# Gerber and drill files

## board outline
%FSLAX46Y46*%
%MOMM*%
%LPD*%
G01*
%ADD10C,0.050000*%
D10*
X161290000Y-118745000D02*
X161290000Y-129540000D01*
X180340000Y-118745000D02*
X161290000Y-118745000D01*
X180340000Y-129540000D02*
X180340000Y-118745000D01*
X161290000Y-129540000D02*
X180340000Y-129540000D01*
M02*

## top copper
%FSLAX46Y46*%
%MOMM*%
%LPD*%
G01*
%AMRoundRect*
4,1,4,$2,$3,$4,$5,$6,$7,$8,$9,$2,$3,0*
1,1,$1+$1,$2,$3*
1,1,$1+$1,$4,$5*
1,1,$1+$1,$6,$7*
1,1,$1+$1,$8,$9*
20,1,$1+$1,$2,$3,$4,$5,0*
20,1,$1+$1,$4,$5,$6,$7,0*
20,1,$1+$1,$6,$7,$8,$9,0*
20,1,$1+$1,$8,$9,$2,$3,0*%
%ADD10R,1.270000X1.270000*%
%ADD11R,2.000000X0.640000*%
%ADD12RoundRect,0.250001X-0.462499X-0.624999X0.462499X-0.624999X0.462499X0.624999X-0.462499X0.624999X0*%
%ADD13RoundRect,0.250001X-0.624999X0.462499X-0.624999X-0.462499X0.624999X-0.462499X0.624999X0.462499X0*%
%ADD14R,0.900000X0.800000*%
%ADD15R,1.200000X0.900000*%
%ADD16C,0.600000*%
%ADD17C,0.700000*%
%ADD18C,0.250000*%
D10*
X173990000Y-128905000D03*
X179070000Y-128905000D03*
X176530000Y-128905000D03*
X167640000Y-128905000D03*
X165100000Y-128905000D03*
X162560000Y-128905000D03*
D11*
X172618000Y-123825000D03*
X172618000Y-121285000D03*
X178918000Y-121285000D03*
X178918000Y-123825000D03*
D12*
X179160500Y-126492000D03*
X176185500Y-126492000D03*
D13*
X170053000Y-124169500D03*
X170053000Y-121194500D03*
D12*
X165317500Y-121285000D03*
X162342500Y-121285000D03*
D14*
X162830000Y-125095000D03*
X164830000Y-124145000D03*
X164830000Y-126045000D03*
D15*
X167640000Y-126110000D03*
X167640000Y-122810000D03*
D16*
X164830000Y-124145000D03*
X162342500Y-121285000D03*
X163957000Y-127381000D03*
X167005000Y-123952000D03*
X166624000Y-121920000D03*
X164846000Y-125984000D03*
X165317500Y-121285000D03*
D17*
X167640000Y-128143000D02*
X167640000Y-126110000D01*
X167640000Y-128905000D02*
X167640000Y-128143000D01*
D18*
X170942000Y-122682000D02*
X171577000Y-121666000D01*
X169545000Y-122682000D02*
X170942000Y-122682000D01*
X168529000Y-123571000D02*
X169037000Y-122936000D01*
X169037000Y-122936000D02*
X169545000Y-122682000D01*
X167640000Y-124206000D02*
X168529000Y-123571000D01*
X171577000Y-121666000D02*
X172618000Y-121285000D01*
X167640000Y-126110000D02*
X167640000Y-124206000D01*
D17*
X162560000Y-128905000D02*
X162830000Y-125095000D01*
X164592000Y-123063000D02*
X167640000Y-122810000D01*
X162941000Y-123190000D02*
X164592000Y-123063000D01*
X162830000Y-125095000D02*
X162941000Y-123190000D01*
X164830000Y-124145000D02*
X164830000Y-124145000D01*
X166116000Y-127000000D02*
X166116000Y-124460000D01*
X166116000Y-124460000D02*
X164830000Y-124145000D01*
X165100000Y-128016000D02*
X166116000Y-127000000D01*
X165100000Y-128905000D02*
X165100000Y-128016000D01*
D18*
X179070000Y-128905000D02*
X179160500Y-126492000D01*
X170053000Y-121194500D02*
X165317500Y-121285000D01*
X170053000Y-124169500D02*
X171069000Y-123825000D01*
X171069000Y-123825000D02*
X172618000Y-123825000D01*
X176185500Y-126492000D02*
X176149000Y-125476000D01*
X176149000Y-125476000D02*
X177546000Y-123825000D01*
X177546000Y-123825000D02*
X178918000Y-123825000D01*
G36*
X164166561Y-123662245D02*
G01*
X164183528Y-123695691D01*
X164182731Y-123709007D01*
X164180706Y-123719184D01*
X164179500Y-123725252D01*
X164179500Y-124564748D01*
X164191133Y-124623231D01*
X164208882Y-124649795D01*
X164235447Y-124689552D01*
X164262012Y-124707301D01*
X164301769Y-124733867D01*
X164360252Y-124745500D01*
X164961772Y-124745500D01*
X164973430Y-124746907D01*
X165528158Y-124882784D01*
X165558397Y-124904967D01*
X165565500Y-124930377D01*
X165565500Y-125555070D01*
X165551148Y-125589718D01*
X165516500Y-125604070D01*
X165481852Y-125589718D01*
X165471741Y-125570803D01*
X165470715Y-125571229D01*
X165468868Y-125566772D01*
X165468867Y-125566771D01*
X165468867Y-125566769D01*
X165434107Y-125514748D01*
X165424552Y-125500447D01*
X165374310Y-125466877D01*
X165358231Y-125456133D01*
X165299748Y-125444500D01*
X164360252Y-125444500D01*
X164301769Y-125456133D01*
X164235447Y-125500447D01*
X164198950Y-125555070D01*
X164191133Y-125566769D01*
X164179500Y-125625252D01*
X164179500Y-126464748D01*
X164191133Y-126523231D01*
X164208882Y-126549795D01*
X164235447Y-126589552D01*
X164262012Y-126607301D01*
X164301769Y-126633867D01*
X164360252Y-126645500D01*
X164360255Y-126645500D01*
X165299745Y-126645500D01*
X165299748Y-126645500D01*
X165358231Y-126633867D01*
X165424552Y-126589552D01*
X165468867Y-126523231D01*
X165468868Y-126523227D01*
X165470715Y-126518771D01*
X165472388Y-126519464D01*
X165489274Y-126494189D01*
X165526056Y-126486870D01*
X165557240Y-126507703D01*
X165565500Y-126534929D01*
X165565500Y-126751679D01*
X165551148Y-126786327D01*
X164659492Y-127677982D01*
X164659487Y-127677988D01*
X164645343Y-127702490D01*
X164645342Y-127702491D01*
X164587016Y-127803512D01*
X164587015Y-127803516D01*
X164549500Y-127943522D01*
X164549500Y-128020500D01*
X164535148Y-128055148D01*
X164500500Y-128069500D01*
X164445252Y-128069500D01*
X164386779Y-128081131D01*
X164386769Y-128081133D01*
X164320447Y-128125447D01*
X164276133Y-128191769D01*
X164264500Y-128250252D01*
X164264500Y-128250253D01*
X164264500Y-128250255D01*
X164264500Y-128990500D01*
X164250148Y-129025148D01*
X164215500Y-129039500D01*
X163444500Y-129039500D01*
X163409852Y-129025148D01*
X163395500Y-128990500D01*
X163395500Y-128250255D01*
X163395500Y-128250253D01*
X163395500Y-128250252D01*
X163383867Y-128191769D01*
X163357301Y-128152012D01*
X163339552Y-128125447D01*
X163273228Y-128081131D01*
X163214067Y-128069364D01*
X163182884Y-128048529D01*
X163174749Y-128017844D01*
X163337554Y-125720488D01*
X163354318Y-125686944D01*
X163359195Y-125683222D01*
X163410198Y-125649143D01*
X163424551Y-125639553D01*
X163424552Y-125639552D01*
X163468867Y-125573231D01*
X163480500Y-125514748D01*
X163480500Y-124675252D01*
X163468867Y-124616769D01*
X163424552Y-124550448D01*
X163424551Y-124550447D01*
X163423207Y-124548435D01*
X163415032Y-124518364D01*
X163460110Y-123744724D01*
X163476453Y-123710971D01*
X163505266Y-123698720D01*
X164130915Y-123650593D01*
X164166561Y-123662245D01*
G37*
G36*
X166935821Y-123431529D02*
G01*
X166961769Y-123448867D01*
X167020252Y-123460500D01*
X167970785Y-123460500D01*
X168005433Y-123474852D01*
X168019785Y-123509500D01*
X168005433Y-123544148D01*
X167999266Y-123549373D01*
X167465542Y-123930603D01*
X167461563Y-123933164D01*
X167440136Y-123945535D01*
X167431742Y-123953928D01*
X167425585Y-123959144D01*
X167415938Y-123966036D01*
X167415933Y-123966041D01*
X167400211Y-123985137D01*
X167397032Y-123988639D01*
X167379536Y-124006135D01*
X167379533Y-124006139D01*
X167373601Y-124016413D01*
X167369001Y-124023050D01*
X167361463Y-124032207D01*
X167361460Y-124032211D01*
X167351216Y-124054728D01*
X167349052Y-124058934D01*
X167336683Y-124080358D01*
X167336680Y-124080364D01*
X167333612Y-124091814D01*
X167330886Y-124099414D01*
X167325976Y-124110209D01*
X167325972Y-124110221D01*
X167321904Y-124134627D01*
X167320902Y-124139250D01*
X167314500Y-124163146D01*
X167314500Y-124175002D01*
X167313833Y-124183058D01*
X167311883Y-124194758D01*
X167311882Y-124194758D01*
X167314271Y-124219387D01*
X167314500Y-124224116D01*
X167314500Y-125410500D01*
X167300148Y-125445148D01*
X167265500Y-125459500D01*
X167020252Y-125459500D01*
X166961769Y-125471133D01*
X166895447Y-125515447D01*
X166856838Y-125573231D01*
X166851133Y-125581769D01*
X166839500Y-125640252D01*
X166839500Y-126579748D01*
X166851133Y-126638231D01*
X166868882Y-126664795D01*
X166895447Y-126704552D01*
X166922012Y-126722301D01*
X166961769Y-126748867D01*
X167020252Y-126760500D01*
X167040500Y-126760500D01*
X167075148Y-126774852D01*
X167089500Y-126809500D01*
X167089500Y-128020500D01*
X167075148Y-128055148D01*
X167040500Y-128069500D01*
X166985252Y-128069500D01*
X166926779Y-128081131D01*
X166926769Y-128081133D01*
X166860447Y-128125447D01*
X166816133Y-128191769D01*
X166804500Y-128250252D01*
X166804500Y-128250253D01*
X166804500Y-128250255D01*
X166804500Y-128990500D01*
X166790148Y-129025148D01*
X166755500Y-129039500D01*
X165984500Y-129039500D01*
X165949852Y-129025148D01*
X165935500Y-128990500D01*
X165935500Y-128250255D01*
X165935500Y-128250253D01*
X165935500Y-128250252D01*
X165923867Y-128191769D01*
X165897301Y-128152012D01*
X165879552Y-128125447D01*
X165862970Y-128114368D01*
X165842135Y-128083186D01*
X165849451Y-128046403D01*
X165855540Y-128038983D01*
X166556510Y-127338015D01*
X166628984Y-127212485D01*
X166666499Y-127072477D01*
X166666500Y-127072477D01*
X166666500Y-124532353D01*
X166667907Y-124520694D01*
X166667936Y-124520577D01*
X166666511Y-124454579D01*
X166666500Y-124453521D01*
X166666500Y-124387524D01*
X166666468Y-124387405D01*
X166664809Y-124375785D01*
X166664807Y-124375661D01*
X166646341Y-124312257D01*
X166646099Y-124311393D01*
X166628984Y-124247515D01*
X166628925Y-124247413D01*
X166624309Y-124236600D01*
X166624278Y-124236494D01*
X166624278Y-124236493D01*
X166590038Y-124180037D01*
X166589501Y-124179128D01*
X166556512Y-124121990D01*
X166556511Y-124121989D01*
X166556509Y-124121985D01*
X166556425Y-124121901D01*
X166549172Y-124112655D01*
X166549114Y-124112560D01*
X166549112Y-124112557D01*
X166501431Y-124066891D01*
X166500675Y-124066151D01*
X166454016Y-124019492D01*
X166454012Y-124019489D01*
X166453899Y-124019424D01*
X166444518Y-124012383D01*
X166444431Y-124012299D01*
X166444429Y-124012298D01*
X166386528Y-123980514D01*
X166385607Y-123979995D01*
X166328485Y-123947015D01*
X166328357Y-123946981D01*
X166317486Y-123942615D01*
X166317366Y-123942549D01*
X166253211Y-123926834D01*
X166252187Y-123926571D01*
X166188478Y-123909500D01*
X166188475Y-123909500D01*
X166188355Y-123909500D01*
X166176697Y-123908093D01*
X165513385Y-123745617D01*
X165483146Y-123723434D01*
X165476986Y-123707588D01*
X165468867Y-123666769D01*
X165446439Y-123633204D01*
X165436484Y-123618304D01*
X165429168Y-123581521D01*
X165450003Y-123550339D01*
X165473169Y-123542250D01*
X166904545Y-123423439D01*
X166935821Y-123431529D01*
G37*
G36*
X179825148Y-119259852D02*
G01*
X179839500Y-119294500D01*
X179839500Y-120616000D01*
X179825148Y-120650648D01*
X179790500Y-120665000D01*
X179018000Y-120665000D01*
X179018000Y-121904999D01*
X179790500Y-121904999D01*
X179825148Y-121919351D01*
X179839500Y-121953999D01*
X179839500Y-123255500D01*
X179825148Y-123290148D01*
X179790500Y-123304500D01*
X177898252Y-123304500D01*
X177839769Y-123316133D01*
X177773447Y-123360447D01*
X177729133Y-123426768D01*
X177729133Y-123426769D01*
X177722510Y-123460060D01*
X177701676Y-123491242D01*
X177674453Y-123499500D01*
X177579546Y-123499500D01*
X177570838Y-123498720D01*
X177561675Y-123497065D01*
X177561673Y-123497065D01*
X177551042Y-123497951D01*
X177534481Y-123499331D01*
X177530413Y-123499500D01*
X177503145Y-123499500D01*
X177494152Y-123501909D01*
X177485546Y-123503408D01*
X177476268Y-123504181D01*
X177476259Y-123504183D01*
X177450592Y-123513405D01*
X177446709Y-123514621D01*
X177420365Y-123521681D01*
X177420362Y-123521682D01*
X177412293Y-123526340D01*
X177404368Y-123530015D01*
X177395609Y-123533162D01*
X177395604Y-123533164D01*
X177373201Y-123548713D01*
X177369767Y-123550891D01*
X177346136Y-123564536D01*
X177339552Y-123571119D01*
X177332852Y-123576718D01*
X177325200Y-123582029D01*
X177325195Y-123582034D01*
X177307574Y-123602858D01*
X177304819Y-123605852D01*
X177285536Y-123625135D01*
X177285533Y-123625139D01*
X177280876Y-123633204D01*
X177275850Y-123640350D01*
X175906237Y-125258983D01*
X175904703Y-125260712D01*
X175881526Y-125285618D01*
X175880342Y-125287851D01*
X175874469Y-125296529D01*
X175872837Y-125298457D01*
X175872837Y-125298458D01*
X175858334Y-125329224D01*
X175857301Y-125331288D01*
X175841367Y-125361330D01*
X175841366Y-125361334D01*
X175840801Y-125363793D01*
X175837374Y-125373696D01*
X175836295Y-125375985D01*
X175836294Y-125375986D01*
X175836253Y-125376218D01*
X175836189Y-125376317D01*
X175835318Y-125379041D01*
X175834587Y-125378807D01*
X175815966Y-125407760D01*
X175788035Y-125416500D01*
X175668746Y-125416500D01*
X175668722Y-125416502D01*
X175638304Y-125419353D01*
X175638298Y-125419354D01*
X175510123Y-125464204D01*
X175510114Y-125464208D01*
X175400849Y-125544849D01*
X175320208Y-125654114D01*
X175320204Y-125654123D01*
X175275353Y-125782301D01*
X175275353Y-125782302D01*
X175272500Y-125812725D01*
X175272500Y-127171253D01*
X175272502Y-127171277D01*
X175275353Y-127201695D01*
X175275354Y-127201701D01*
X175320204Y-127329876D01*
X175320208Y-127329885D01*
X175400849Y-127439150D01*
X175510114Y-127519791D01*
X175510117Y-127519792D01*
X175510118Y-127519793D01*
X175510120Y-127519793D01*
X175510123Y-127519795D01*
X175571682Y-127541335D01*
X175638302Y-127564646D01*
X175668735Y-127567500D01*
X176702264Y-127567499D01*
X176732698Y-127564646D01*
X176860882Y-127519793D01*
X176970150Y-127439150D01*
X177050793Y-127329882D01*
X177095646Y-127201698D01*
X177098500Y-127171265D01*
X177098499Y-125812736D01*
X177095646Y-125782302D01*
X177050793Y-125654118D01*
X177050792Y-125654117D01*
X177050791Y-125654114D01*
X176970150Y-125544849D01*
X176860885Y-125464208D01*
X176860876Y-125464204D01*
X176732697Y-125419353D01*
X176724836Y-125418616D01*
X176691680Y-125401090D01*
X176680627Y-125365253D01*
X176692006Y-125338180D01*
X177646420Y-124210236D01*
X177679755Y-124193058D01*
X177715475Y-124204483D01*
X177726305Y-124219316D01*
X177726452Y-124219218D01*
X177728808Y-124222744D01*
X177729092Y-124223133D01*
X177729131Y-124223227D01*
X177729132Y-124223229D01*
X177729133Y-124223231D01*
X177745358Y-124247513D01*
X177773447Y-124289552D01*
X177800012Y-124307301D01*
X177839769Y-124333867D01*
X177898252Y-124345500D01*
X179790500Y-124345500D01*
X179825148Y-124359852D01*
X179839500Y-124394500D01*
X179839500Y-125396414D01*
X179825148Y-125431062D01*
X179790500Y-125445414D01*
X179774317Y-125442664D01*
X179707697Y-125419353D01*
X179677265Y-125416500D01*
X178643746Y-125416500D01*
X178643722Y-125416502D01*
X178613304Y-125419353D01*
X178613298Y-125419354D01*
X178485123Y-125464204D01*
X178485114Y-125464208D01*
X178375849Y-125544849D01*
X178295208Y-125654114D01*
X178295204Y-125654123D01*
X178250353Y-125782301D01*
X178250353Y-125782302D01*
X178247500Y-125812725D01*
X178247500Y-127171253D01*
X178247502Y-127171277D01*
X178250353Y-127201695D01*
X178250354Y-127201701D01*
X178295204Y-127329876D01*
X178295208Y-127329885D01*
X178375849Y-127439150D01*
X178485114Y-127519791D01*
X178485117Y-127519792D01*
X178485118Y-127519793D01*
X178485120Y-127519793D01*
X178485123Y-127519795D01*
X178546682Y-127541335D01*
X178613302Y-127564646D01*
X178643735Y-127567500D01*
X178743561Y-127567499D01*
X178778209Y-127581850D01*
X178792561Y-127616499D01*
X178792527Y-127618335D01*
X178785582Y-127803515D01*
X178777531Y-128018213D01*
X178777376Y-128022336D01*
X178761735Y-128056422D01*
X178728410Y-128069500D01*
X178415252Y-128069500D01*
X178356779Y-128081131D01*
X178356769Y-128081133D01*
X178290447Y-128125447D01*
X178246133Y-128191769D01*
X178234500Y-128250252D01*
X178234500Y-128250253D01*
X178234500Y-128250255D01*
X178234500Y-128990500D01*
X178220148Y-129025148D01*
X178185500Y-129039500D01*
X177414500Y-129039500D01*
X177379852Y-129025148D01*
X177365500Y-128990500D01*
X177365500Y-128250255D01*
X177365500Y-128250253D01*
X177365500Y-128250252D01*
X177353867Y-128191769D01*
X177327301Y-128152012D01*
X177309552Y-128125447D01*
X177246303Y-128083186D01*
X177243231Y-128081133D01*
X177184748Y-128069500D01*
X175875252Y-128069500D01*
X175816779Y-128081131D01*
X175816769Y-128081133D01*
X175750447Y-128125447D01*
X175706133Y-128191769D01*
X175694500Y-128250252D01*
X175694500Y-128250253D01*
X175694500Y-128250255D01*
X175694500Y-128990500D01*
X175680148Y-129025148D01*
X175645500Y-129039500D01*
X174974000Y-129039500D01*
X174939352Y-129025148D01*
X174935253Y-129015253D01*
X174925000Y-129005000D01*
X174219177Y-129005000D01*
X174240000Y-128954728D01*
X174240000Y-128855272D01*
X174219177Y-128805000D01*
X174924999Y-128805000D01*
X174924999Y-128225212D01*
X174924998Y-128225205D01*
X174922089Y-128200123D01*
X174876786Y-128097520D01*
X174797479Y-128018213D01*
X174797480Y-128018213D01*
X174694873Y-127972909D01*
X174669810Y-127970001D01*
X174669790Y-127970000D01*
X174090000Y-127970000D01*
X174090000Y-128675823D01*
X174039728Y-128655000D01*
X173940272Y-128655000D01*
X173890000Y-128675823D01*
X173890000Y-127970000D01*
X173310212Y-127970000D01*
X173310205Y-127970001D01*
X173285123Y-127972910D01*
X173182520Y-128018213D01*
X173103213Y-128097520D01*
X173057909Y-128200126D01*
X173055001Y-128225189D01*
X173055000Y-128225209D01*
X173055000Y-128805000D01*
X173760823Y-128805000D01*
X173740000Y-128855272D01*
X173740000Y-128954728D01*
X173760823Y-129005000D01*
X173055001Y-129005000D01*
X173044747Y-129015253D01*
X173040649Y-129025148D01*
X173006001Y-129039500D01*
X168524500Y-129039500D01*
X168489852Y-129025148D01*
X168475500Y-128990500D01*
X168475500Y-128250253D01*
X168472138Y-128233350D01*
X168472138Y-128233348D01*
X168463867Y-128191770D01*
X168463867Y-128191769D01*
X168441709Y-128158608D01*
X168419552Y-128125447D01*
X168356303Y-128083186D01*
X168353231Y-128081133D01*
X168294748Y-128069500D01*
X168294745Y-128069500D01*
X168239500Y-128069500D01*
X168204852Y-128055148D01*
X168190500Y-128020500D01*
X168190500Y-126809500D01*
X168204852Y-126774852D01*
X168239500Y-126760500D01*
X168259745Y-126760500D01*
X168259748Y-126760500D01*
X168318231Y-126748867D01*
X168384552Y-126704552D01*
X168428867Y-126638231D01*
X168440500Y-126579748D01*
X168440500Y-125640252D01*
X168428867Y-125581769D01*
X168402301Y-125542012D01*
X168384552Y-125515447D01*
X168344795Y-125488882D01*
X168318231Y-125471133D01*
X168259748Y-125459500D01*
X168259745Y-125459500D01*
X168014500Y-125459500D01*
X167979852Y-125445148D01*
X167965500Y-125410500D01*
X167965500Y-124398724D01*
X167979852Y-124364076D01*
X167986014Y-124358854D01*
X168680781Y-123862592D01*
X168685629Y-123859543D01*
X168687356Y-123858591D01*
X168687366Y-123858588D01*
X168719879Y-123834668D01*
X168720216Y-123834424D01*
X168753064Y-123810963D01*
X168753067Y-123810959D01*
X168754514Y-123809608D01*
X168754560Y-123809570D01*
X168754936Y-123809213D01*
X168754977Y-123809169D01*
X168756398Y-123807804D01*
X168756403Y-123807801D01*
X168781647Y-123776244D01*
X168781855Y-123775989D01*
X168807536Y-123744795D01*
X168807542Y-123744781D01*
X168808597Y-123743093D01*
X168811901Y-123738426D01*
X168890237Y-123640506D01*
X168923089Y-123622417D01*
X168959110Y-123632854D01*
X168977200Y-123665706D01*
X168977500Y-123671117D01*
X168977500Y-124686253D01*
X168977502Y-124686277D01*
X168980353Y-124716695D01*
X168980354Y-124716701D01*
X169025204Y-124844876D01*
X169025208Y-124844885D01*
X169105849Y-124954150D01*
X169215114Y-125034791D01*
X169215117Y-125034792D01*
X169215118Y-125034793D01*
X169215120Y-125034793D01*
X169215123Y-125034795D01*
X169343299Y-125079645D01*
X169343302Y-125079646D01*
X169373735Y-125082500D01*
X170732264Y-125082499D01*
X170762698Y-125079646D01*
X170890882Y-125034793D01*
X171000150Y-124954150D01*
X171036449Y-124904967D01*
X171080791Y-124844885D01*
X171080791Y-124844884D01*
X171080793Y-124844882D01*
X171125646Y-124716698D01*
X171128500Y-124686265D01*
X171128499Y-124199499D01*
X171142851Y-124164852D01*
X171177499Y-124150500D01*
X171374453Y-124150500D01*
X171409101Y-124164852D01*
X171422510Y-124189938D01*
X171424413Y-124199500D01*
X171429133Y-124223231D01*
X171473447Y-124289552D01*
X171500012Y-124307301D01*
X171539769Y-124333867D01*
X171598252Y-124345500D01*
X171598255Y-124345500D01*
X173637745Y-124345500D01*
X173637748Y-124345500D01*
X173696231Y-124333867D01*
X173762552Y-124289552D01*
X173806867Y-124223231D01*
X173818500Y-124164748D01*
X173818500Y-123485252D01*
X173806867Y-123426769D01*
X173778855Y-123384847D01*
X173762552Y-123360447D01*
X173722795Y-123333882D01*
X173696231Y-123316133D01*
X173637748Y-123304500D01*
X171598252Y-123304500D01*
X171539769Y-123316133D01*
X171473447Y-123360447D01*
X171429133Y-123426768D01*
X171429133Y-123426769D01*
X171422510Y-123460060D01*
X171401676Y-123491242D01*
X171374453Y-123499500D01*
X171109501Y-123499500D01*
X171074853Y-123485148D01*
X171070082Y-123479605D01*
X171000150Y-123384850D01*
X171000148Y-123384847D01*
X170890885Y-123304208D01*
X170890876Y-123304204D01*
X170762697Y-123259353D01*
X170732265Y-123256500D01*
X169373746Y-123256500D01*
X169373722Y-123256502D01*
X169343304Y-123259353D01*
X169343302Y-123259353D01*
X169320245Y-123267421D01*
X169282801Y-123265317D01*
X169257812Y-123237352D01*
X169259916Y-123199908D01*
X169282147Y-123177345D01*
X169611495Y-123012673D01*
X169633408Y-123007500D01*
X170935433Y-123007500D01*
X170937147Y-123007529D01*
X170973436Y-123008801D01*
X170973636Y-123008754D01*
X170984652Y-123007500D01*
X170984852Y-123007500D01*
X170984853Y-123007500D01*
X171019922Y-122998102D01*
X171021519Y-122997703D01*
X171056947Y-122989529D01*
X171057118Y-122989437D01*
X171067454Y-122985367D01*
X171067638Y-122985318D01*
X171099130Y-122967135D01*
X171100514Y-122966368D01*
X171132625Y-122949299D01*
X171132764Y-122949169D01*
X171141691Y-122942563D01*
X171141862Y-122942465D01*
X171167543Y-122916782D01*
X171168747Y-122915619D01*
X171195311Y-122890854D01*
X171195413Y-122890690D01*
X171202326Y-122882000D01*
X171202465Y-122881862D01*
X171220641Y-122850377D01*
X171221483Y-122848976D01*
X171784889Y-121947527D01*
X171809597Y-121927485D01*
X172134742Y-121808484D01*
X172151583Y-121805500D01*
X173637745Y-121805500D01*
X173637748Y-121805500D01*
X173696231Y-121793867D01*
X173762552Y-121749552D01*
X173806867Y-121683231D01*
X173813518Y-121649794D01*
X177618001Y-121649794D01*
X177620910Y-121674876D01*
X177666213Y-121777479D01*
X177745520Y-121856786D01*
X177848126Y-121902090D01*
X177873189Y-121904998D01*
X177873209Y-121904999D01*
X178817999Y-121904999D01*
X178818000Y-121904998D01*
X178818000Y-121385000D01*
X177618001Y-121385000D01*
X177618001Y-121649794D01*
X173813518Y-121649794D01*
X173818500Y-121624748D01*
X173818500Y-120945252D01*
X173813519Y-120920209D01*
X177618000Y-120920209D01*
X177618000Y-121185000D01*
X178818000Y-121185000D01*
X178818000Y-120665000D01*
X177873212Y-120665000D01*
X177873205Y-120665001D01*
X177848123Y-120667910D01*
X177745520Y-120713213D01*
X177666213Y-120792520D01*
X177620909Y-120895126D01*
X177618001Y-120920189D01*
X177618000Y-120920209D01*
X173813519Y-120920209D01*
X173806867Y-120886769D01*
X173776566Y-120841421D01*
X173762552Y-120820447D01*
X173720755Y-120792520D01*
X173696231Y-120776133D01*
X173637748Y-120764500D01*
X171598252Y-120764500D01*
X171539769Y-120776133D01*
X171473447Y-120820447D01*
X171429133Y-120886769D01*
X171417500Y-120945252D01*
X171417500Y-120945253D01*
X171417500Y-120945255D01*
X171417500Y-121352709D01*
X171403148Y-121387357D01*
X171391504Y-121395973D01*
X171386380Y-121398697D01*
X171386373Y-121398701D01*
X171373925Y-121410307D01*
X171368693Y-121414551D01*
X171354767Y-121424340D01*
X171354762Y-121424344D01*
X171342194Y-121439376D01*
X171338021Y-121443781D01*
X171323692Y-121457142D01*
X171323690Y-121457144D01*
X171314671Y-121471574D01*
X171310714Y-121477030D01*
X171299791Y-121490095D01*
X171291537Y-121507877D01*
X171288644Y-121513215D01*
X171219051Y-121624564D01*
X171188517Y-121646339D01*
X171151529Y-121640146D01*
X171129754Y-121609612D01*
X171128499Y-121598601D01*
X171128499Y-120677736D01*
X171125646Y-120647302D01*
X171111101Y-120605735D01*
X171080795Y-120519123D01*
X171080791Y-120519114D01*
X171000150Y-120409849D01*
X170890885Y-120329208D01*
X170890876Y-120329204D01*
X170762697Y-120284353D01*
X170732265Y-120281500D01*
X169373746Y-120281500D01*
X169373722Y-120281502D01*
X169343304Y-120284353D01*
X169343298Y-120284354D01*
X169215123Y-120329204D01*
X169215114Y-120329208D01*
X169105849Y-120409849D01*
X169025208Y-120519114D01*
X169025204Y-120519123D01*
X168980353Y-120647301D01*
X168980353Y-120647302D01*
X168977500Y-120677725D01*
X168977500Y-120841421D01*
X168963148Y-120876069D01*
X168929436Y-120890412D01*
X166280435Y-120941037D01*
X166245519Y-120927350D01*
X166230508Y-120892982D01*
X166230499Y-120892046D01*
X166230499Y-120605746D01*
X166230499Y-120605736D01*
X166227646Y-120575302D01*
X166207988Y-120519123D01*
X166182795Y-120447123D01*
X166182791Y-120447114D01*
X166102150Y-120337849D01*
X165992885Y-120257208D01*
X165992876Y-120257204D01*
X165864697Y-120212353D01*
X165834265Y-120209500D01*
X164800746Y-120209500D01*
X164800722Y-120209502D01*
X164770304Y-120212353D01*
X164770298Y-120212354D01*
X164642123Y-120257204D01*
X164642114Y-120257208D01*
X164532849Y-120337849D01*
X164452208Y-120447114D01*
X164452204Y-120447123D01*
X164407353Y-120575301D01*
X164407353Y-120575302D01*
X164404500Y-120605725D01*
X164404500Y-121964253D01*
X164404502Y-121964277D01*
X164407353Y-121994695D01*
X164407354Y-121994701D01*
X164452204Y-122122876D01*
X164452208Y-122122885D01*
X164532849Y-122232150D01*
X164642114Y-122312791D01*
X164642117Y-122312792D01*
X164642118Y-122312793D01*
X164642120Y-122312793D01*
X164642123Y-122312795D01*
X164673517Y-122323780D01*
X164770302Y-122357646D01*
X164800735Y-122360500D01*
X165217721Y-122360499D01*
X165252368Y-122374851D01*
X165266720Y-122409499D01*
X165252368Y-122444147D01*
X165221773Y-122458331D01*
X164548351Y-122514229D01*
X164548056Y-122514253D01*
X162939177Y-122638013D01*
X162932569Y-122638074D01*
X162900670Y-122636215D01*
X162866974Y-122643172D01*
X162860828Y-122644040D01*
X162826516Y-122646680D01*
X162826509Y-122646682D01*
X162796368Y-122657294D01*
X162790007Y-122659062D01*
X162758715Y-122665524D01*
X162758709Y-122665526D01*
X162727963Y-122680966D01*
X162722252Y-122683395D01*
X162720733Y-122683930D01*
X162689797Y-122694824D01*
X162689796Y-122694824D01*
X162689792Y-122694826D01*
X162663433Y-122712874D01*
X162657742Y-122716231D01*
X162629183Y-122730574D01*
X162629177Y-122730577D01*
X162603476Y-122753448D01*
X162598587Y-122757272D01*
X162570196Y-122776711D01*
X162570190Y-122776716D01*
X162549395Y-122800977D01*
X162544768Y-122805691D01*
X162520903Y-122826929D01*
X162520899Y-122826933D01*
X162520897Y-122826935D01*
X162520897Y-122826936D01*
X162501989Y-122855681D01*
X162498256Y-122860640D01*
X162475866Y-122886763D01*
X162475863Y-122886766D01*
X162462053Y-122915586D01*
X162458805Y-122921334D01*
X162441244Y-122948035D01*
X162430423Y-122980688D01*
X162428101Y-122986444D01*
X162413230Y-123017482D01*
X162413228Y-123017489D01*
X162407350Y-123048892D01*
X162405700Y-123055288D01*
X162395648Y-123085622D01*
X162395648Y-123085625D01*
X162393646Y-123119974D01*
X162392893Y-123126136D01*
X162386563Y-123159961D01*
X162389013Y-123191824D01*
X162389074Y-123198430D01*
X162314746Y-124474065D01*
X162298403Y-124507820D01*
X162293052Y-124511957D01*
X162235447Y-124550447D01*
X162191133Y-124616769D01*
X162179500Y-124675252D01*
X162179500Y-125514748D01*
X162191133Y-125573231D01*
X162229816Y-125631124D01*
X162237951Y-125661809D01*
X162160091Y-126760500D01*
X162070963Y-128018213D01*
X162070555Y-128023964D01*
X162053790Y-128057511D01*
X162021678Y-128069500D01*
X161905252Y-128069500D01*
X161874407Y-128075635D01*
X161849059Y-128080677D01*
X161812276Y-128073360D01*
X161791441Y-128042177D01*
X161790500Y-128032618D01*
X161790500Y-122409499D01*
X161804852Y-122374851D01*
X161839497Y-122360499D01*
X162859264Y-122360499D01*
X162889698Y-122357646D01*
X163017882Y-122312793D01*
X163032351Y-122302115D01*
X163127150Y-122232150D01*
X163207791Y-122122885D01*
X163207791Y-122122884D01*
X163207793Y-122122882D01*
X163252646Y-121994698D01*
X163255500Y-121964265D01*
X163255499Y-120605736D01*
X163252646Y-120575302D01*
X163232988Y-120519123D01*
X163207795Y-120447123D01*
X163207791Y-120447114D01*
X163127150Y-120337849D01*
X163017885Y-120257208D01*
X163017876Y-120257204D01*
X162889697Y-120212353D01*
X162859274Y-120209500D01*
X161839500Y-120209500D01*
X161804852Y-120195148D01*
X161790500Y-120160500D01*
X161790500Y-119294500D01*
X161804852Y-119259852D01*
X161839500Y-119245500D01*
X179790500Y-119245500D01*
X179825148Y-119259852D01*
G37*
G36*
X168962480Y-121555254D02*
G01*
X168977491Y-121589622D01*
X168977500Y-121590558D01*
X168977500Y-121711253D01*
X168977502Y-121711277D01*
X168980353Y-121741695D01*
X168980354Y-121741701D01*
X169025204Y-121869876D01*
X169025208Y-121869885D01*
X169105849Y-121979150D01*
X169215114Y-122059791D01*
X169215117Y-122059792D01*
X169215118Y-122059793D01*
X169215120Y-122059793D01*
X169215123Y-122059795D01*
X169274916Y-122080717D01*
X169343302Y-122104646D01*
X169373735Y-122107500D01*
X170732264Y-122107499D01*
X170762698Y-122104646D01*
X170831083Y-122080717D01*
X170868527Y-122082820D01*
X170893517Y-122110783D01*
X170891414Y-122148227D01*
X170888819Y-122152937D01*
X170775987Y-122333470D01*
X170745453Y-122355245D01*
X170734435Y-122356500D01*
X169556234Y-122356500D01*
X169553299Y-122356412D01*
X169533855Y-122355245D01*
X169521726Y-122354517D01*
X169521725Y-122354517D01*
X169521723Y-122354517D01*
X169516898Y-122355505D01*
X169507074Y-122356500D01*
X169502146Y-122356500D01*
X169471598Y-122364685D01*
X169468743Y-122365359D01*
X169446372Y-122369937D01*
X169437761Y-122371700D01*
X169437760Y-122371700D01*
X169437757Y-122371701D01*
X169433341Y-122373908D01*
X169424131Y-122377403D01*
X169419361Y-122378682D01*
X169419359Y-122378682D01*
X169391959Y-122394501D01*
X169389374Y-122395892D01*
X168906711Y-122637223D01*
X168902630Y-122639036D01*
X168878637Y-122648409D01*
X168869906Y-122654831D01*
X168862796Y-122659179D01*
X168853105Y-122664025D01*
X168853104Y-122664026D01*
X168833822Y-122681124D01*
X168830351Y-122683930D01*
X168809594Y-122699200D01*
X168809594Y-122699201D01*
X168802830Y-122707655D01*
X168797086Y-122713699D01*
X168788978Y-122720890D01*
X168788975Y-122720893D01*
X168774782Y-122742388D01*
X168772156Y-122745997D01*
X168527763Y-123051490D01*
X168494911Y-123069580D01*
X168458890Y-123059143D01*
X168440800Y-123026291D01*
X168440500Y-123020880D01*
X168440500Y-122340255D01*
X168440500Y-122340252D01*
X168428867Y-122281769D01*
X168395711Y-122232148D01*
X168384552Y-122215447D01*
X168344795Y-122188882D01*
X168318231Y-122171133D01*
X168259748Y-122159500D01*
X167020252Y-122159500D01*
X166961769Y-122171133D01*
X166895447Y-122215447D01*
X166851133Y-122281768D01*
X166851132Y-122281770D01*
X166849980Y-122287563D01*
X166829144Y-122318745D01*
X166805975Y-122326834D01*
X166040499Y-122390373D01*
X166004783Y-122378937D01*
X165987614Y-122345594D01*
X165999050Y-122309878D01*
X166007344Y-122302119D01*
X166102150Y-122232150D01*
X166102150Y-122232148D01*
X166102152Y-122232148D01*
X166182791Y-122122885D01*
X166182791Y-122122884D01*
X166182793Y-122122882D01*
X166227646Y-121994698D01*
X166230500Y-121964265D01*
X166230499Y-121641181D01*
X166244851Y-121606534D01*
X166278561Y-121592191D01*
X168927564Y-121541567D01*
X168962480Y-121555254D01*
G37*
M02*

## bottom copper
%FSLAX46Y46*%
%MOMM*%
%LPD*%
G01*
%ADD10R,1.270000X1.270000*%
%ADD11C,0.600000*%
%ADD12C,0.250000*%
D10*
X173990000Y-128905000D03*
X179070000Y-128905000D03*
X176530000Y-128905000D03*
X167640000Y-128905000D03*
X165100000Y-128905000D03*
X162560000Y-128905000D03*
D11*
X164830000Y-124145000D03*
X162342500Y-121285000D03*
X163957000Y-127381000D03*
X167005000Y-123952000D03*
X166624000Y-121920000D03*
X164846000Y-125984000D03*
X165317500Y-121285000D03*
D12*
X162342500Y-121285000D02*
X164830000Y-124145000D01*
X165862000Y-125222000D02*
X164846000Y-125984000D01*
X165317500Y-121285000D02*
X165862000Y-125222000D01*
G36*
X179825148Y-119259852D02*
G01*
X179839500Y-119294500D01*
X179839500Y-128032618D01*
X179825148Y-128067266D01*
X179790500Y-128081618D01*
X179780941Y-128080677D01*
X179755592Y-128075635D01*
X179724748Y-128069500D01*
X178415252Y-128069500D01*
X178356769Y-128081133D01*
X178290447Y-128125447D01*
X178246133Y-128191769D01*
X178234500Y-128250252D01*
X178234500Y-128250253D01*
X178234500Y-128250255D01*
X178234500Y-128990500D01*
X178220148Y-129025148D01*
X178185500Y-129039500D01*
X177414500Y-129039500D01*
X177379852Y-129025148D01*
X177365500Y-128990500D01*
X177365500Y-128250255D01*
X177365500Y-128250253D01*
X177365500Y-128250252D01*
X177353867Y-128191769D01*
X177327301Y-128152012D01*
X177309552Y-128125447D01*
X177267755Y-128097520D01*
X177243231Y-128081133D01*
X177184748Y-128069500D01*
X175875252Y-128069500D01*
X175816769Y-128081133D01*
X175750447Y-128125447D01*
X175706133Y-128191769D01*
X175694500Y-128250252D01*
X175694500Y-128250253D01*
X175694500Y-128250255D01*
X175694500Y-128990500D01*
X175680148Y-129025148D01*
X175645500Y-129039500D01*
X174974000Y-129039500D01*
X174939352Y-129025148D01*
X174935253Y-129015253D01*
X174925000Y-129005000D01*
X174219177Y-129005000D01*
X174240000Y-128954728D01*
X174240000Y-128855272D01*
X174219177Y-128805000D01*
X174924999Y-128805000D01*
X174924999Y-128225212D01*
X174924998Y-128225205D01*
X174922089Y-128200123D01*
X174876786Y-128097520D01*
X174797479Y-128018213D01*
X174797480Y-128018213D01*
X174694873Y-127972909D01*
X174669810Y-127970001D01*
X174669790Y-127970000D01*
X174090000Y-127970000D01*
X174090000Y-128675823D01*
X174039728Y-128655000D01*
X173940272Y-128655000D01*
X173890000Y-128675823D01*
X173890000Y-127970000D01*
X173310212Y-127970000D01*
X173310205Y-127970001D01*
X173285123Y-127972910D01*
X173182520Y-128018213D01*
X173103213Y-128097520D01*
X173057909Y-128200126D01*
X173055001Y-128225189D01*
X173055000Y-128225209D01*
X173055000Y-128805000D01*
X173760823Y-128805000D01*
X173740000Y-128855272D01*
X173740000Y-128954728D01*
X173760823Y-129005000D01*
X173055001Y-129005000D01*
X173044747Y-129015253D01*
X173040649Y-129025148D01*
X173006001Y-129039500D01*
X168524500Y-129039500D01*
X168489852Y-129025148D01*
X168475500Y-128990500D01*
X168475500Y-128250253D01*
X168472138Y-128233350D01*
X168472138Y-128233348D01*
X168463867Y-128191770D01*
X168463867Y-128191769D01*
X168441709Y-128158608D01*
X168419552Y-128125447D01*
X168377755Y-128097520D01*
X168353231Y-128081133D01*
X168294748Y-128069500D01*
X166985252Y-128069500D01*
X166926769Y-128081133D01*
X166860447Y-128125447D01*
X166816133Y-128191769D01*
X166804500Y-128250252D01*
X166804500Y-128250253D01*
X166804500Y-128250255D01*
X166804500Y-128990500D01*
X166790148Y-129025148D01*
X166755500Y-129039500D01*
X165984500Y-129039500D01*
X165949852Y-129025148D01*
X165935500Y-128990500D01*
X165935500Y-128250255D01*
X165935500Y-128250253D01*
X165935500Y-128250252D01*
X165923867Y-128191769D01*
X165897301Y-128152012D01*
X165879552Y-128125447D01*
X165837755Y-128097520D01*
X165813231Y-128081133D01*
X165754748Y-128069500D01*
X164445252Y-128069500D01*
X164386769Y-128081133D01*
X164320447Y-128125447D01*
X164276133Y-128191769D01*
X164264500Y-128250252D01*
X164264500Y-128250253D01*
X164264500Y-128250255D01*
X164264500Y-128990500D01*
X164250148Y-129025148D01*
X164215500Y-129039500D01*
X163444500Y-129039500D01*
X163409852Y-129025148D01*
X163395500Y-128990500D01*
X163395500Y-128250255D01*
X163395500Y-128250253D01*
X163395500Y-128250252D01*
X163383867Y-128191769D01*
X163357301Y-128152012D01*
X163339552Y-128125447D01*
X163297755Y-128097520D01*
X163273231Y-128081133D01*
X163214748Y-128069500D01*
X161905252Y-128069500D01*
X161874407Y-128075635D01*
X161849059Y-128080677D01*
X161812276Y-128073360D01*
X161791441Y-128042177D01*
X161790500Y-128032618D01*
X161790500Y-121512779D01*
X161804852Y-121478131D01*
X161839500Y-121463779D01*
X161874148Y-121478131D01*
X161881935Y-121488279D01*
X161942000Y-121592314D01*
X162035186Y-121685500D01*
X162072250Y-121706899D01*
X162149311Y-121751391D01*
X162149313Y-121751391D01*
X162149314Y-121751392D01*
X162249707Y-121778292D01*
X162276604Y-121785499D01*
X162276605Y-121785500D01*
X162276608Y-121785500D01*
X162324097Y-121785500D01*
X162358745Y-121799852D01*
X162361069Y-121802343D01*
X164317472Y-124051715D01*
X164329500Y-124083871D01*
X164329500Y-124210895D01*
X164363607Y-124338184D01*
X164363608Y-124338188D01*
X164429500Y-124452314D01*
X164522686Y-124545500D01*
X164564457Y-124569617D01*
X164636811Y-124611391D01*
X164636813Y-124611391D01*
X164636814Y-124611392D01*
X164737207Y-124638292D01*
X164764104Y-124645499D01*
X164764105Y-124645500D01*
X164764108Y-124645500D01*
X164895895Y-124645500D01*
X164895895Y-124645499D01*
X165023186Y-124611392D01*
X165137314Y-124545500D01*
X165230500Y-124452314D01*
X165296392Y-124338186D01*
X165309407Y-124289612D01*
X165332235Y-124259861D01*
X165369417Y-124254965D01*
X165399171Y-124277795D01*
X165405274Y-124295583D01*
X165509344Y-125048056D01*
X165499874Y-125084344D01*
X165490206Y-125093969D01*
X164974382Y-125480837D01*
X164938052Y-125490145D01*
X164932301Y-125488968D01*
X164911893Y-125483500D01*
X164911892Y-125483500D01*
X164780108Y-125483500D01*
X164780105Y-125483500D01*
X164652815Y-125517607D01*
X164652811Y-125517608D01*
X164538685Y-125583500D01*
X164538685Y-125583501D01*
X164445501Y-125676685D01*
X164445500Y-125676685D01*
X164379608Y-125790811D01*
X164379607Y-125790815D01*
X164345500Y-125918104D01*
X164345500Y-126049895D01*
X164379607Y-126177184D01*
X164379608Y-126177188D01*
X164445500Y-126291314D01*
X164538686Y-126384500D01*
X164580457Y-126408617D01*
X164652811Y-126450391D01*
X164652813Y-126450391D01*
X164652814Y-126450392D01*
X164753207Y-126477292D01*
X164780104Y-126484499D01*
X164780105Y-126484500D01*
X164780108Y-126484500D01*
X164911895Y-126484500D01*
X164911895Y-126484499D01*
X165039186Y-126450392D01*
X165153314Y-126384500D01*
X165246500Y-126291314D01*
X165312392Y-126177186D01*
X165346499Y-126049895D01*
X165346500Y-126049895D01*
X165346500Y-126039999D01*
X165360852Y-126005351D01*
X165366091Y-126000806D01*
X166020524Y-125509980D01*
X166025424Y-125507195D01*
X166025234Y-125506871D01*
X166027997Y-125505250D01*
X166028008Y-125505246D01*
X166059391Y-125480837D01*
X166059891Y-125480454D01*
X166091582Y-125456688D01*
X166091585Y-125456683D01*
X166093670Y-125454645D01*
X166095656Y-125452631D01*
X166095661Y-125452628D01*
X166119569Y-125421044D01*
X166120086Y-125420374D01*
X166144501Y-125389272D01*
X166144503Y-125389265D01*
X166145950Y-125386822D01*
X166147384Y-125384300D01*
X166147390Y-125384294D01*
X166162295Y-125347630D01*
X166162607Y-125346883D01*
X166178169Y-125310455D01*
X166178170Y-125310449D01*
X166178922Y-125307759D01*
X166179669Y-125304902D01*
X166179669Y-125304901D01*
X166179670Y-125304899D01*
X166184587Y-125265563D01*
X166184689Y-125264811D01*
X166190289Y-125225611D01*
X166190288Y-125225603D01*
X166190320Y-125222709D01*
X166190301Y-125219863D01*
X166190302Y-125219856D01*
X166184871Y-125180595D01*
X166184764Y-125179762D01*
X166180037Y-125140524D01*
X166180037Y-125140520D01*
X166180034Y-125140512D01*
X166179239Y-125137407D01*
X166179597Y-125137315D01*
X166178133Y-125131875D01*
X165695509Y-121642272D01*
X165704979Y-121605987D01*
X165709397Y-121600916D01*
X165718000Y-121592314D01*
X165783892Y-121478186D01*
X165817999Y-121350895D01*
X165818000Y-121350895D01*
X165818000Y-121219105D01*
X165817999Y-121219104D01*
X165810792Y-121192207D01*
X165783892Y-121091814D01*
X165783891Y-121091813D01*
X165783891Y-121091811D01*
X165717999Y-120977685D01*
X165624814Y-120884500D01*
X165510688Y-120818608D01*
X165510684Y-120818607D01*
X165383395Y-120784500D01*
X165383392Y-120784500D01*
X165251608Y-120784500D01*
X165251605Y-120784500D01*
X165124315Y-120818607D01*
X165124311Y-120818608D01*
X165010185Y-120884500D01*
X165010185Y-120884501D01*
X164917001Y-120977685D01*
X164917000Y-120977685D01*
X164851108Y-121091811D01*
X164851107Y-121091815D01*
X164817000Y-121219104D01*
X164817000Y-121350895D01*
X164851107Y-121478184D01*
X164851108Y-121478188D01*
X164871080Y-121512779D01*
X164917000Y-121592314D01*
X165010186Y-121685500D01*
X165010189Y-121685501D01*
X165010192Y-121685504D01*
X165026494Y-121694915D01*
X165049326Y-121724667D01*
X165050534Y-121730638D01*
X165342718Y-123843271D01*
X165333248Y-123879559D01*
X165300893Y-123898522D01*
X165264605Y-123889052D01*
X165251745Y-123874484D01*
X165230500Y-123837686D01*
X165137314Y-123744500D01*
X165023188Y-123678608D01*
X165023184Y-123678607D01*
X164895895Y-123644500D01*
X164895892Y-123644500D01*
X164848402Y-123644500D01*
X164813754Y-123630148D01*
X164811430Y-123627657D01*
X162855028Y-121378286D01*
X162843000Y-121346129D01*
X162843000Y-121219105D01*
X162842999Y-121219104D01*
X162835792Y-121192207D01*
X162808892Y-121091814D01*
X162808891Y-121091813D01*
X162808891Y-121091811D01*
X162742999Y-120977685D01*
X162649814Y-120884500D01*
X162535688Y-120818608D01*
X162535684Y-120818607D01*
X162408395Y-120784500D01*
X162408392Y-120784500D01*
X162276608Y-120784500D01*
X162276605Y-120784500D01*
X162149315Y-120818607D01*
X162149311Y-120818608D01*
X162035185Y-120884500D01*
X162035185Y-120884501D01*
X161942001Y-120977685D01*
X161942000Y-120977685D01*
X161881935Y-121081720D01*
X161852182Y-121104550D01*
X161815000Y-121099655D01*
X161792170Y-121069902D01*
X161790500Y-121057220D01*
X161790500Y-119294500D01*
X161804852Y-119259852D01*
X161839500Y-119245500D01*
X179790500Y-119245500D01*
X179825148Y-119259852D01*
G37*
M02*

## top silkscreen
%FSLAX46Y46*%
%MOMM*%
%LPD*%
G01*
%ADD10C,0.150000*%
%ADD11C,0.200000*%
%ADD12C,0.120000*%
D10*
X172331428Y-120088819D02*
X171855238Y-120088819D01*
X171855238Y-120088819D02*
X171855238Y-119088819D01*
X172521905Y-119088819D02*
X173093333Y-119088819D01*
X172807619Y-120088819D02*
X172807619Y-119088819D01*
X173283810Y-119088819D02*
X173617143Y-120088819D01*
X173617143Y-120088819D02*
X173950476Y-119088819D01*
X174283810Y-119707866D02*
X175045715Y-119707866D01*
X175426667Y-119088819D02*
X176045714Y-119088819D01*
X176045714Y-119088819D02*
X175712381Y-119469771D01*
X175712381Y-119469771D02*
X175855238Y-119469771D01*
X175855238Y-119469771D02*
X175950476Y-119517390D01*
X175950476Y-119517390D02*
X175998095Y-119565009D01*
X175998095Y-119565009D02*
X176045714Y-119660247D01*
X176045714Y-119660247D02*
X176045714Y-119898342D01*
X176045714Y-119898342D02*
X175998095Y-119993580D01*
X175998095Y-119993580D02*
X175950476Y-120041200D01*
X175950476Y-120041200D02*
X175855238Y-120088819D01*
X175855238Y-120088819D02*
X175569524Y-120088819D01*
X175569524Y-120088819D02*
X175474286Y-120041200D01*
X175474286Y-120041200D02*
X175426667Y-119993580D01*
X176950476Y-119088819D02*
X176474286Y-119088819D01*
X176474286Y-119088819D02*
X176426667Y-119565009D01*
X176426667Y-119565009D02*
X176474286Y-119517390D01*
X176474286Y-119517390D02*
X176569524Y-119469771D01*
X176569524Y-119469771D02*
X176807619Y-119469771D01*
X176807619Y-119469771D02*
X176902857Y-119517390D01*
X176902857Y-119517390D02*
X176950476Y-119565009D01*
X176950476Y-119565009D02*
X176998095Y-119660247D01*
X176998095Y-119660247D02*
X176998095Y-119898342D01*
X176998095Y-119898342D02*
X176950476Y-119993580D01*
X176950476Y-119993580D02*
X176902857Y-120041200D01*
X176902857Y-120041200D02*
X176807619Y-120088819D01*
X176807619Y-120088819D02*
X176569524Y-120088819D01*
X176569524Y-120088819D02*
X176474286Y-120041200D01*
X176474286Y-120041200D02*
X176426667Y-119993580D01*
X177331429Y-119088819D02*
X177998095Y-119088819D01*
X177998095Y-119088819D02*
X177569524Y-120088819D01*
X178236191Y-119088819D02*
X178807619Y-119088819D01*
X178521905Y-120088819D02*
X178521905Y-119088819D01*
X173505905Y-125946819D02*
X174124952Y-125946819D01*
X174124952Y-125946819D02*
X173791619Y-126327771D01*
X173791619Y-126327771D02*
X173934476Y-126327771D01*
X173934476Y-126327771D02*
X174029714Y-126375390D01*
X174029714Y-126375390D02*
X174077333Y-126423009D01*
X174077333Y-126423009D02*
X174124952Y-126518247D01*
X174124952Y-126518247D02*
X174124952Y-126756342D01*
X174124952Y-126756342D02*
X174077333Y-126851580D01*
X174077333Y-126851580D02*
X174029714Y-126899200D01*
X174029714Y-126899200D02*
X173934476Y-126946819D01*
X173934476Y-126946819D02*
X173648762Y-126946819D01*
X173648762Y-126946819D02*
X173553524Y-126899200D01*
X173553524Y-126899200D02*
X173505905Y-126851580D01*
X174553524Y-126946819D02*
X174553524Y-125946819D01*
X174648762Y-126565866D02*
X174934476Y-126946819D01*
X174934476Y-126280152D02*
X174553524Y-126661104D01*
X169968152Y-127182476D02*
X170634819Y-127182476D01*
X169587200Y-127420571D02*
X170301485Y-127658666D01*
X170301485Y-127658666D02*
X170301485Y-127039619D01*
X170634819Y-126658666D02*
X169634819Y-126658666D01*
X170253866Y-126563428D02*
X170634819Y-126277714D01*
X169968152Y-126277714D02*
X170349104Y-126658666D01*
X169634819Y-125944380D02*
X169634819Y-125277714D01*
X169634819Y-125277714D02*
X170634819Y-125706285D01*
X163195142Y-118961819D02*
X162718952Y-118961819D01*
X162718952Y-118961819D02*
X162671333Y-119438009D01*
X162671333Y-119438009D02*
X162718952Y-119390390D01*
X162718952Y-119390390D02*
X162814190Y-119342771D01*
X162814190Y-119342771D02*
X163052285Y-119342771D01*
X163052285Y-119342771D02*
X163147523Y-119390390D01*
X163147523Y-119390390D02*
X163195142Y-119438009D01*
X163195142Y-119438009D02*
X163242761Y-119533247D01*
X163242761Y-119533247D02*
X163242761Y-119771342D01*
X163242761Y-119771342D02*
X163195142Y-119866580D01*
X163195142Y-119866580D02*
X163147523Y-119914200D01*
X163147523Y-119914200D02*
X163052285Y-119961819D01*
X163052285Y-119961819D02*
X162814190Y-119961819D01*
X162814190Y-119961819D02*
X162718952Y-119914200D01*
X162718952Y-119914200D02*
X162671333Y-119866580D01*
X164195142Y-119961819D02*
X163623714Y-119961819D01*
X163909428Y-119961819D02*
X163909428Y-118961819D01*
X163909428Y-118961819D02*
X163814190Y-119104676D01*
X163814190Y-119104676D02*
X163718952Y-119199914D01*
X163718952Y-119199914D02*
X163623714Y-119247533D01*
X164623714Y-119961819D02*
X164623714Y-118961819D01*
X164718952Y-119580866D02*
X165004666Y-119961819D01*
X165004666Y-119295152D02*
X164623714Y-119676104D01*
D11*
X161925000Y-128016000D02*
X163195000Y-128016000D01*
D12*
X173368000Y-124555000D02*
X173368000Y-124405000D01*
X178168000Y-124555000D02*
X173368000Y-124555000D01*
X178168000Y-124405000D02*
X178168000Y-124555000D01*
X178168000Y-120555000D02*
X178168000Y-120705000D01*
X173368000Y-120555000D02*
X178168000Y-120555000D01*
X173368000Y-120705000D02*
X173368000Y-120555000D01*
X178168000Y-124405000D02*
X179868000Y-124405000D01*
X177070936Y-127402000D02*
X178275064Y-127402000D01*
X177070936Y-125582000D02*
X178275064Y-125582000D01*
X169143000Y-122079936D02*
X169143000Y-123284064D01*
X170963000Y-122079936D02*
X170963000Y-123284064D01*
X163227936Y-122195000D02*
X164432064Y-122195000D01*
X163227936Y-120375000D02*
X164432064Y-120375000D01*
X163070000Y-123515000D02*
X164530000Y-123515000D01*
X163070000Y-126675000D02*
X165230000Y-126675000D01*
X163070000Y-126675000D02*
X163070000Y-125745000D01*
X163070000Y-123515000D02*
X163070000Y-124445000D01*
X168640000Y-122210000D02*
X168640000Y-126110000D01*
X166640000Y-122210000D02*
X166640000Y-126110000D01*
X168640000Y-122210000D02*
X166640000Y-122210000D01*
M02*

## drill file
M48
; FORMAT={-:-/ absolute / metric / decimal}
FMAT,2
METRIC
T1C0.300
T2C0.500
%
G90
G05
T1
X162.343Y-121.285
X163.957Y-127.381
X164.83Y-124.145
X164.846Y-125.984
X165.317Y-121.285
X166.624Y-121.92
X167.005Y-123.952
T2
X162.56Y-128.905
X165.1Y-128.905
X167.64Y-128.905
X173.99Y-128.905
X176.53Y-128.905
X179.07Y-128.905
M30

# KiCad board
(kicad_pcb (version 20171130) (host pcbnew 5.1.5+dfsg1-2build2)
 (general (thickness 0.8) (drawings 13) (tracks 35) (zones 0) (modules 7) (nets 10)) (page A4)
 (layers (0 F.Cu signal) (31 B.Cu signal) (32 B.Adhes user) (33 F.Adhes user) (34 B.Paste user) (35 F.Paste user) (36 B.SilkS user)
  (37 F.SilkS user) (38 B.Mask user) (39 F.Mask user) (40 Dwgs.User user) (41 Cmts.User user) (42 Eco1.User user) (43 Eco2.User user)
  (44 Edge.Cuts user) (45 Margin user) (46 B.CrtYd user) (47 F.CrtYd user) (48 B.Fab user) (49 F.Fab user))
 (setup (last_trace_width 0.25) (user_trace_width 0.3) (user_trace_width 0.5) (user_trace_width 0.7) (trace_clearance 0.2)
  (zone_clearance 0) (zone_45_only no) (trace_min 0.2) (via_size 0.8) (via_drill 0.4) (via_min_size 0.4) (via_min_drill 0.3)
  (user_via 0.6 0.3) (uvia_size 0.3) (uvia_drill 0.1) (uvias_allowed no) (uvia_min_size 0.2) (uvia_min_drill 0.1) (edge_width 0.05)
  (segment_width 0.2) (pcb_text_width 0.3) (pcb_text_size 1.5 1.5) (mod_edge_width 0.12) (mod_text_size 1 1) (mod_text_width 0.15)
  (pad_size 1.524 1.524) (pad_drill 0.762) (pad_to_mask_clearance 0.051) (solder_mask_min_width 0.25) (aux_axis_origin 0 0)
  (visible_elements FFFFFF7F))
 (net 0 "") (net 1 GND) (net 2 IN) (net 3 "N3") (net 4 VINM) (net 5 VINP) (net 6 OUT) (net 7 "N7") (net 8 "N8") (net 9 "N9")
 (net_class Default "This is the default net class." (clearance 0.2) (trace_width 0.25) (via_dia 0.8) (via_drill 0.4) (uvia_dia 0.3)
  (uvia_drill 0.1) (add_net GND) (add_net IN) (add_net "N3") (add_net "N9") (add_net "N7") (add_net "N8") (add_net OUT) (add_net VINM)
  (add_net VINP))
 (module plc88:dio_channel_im (layer F.Cu) (at 169.545 126.365)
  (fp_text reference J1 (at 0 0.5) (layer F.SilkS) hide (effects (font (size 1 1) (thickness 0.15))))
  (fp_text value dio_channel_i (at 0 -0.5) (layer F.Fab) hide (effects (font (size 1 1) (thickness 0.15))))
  (fp_line (start -7.62 1.651) (end -6.35 1.651) (layer F.SilkS) (width 0.2))
  (pad 4 thru_hole rect (at 4.445 2.54) (size 1.27 1.27) (drill 0.5) (layers *.Cu *.Mask) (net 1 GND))
  (pad 6 thru_hole rect (at 9.525 2.54) (size 1.27 1.27) (drill 0.5) (layers *.Cu *.Mask) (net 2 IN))
  (pad 5 thru_hole rect (at 6.985 2.54) (size 1.27 1.27) (drill 0.5) (layers *.Cu *.Mask) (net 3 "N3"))
  (pad 3 thru_hole rect (at -1.905 2.54) (size 1.27 1.27) (drill 0.5) (layers *.Cu *.Mask) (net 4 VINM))
  (pad 2 thru_hole rect (at -4.445 2.54) (size 1.27 1.27) (drill 0.5) (layers *.Cu *.Mask) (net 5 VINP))
  (pad 1 thru_hole rect (at -6.985 2.54) (size 1.27 1.27) (drill 0.5) (layers *.Cu *.Mask) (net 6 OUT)))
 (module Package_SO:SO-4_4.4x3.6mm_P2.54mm (layer F.Cu) (at 175.768 122.555 180)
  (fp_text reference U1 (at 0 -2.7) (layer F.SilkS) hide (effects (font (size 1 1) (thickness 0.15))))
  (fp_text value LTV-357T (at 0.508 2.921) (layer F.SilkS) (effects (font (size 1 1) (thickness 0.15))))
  (fp_line (start 2.4 -2) (end 2.4 -1.85) (layer F.SilkS) (width 0.12))
  (fp_line (start -2.4 -2) (end 2.4 -2) (layer F.SilkS) (width 0.12))
  (fp_line (start -2.4 -1.85) (end -2.4 -2) (layer F.SilkS) (width 0.12))
  (fp_line (start -2.4 2) (end -2.4 1.85) (layer F.SilkS) (width 0.12))
  (fp_line (start 2.4 2) (end -2.4 2) (layer F.SilkS) (width 0.12))
  (fp_line (start 2.4 1.85) (end 2.4 2) (layer F.SilkS) (width 0.12))
  (fp_line (start -2.4 -1.85) (end -4.1 -1.85) (layer F.SilkS) (width 0.12))
  (pad 4 smd rect (at 3.15 -1.27 180) (size 2 0.64) (layers F.Cu F.Paste F.Mask) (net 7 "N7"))
  (pad 3 smd rect (at 3.15 1.27 180) (size 2 0.64) (layers F.Cu F.Paste F.Mask) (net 4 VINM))
  (pad 2 smd rect (at -3.15 1.27 180) (size 2 0.64) (layers F.Cu F.Paste F.Mask) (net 1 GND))
  (pad 1 smd rect (at -3.15 -1.27 180) (size 2 0.64) (layers F.Cu F.Paste F.Mask) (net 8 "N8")))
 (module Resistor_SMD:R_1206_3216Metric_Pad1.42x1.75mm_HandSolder (layer F.Cu) (at 177.673 126.492)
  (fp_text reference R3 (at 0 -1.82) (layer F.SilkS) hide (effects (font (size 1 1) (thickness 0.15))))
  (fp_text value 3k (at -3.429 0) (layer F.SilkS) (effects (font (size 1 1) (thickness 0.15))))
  (fp_line (start -0.602064 0.91) (end 0.602064 0.91) (layer F.SilkS) (width 0.12))
  (fp_line (start -0.602064 -0.91) (end 0.602064 -0.91) (layer F.SilkS) (width 0.12))
  (pad 2 smd roundrect (at 1.4875 0) (size 1.425 1.75) (layers F.Cu F.Paste F.Mask) (roundrect_rratio 0.175439) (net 2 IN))
  (pad 1 smd roundrect (at -1.4875 0) (size 1.425 1.75) (layers F.Cu F.Paste F.Mask) (roundrect_rratio 0.175439) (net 8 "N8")))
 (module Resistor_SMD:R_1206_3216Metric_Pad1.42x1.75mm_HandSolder (layer F.Cu) (at 170.053 122.682 270)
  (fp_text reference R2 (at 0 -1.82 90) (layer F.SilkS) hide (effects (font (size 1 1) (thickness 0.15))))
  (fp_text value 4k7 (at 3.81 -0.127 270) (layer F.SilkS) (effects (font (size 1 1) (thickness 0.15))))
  (fp_line (start -0.602064 0.91) (end 0.602064 0.91) (layer F.SilkS) (width 0.12))
  (fp_line (start -0.602064 -0.91) (end 0.602064 -0.91) (layer F.SilkS) (width 0.12))
  (pad 2 smd roundrect (at 1.4875 0 270) (size 1.425 1.75) (layers F.Cu F.Paste F.Mask) (roundrect_rratio 0.175439) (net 7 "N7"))
  (pad 1 smd roundrect (at -1.4875 0 270) (size 1.425 1.75) (layers F.Cu F.Paste F.Mask) (roundrect_rratio 0.175439) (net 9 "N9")))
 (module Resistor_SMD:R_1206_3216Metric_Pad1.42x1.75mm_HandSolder (layer F.Cu) (at 163.83 121.285)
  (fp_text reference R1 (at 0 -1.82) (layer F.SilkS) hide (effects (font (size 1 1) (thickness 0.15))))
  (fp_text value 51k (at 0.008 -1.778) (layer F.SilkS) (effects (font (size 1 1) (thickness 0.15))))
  (fp_line (start -0.602064 0.91) (end 0.602064 0.91) (layer F.SilkS) (width 0.12))
  (fp_line (start -0.602064 -0.91) (end 0.602064 -0.91) (layer F.SilkS) (width 0.12))
  (pad 2 smd roundrect (at 1.4875 0) (size 1.425 1.75) (layers F.Cu F.Paste F.Mask) (roundrect_rratio 0.175439) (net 9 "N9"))
  (pad 1 smd roundrect (at -1.4875 0) (size 1.425 1.75) (layers F.Cu F.Paste F.Mask) (roundrect_rratio 0.175439) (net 5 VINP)))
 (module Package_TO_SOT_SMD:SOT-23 (layer F.Cu) (at 163.83 125.095 180)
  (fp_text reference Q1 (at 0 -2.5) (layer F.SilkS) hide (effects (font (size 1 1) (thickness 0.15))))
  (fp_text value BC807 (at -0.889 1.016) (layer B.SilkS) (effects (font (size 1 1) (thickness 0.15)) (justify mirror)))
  (fp_line (start 0.76 1.58) (end -0.7 1.58) (layer F.SilkS) (width 0.12))
  (fp_line (start 0.76 -1.58) (end -1.4 -1.58) (layer F.SilkS) (width 0.12))
  (fp_line (start 0.76 -1.58) (end 0.76 -0.65) (layer F.SilkS) (width 0.12))
  (fp_line (start 0.76 1.58) (end 0.76 0.65) (layer F.SilkS) (width 0.12))
  (pad 3 smd rect (at 1 0 180) (size 0.9 0.8) (layers F.Cu F.Paste F.Mask) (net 6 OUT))
  (pad 2 smd rect (at -1 0.95 180) (size 0.9 0.8) (layers F.Cu F.Paste F.Mask) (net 5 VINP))
  (pad 1 smd rect (at -1 -0.95 180) (size 0.9 0.8) (layers F.Cu F.Paste F.Mask) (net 9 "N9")))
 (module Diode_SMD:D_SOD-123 (layer F.Cu) (at 167.64 124.46 270)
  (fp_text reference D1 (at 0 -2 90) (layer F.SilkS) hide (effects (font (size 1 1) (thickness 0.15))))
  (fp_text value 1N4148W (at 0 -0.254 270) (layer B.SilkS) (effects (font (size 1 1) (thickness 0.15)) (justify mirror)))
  (fp_line (start -2.25 -1) (end 1.65 -1) (layer F.SilkS) (width 0.12))
  (fp_line (start -2.25 1) (end 1.65 1) (layer F.SilkS) (width 0.12))
  (fp_line (start -2.25 -1) (end -2.25 1) (layer F.SilkS) (width 0.12))
  (pad 2 smd rect (at 1.65 0 270) (size 0.9 1.2) (layers F.Cu F.Paste F.Mask) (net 4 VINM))
  (pad 1 smd rect (at -1.65 0 270) (size 0.9 1.2) (layers F.Cu F.Paste F.Mask) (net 6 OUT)))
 (gr_line (start 161.29 118.745) (end 161.29 129.54) (layer Edge.Cuts) (width 0.05))
 (gr_line (start 180.34 118.745) (end 161.29 118.745) (layer Edge.Cuts) (width 0.05))
 (gr_line (start 180.34 129.54) (end 180.34 118.745) (layer Edge.Cuts) (width 0.05))
 (gr_line (start 161.29 129.54) (end 180.34 129.54) (layer Edge.Cuts) (width 0.05))
 (segment (start 167.64 128.143) (end 167.64 126.11) (width 0.7) (layer F.Cu) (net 4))
 (segment (start 167.64 128.905) (end 167.64 128.143) (width 0.7) (layer F.Cu) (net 4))
 (segment (start 170.942 122.682) (end 171.577 121.666) (width 0.25) (layer F.Cu) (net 4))
 (segment (start 169.545 122.682) (end 170.942 122.682) (width 0.25) (layer F.Cu) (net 4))
 (segment (start 168.529 123.571) (end 169.037 122.936) (width 0.25) (layer F.Cu) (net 4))
 (segment (start 169.037 122.936) (end 169.545 122.682) (width 0.25) (layer F.Cu) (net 4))
 (segment (start 167.64 124.206) (end 168.529 123.571) (width 0.25) (layer F.Cu) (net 4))
 (segment (start 171.577 121.666) (end 172.618 121.285) (width 0.25) (layer F.Cu) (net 4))
 (segment (start 167.64 126.11) (end 167.64 124.206) (width 0.25) (layer F.Cu) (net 4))
 (segment (start 162.56 128.905) (end 162.83 125.095) (width 0.7) (layer F.Cu) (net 6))
 (segment (start 164.592 123.063) (end 167.64 122.81) (width 0.7) (layer F.Cu) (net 6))
 (segment (start 162.941 123.19) (end 164.592 123.063) (width 0.7) (layer F.Cu) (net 6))
 (segment (start 162.83 125.095) (end 162.941 123.19) (width 0.7) (layer F.Cu) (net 6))
 (segment (start 164.83 124.145) (end 164.83 124.145) (width 0.7) (layer F.Cu) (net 5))
 (via (at 164.83 124.145) (size 0.6) (drill 0.3) (layers F.Cu B.Cu) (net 5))
 (segment (start 166.116 127) (end 166.116 124.46) (width 0.7) (layer F.Cu) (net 5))
 (segment (start 166.116 124.46) (end 164.83 124.145) (width 0.7) (layer F.Cu) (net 5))
 (segment (start 165.1 128.016) (end 166.116 127) (width 0.7) (layer F.Cu) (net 5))
 (segment (start 165.1 128.905) (end 165.1 128.016) (width 0.7) (layer F.Cu) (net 5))
 (segment (start 162.3425 121.285) (end 164.83 124.145) (width 0.25) (layer B.Cu) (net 5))
 (via (at 162.3425 121.285) (size 0.6) (drill 0.3) (layers F.Cu B.Cu) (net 5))
 (segment (start 179.07 128.905) (end 179.1605 126.492) (width 0.25) (layer F.Cu) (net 2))
 (via (at 163.957 127.381) (size 0.6) (drill 0.3) (layers F.Cu B.Cu) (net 1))
 (via (at 167.005 123.952) (size 0.6) (drill 0.3) (layers F.Cu B.Cu) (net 1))
 (via (at 166.624 121.92) (size 0.6) (drill 0.3) (layers F.Cu B.Cu) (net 1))
 (via (at 164.846 125.984) (size 0.6) (drill 0.3) (layers F.Cu B.Cu) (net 9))
 (segment (start 165.862 125.222) (end 164.846 125.984) (width 0.25) (layer B.Cu) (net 9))
 (segment (start 165.3175 121.285) (end 165.862 125.222) (width 0.25) (layer B.Cu) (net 9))
 (via (at 165.3175 121.285) (size 0.6) (drill 0.3) (layers F.Cu B.Cu) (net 9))
 (segment (start 170.053 121.1945) (end 165.3175 121.285) (width 0.25) (layer F.Cu) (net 9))
 (segment (start 170.053 124.1695) (end 171.069 123.825) (width 0.25) (layer F.Cu) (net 7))
 (segment (start 171.069 123.825) (end 172.618 123.825) (width 0.25) (layer F.Cu) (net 7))
 (segment (start 176.1855 126.492) (end 176.149 125.476) (width 0.25) (layer F.Cu) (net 8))
 (segment (start 176.149 125.476) (end 177.546 123.825) (width 0.25) (layer F.Cu) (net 8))
 (segment (start 177.546 123.825) (end 178.918 123.825) (width 0.25) (layer F.Cu) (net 8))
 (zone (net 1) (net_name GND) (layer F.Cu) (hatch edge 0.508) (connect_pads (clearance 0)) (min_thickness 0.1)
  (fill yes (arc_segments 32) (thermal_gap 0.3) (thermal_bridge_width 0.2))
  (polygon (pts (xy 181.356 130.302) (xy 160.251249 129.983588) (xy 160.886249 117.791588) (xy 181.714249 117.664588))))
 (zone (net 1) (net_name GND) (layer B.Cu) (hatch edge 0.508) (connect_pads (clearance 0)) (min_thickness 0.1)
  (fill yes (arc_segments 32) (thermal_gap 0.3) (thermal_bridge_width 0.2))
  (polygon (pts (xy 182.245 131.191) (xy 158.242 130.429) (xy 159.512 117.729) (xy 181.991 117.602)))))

